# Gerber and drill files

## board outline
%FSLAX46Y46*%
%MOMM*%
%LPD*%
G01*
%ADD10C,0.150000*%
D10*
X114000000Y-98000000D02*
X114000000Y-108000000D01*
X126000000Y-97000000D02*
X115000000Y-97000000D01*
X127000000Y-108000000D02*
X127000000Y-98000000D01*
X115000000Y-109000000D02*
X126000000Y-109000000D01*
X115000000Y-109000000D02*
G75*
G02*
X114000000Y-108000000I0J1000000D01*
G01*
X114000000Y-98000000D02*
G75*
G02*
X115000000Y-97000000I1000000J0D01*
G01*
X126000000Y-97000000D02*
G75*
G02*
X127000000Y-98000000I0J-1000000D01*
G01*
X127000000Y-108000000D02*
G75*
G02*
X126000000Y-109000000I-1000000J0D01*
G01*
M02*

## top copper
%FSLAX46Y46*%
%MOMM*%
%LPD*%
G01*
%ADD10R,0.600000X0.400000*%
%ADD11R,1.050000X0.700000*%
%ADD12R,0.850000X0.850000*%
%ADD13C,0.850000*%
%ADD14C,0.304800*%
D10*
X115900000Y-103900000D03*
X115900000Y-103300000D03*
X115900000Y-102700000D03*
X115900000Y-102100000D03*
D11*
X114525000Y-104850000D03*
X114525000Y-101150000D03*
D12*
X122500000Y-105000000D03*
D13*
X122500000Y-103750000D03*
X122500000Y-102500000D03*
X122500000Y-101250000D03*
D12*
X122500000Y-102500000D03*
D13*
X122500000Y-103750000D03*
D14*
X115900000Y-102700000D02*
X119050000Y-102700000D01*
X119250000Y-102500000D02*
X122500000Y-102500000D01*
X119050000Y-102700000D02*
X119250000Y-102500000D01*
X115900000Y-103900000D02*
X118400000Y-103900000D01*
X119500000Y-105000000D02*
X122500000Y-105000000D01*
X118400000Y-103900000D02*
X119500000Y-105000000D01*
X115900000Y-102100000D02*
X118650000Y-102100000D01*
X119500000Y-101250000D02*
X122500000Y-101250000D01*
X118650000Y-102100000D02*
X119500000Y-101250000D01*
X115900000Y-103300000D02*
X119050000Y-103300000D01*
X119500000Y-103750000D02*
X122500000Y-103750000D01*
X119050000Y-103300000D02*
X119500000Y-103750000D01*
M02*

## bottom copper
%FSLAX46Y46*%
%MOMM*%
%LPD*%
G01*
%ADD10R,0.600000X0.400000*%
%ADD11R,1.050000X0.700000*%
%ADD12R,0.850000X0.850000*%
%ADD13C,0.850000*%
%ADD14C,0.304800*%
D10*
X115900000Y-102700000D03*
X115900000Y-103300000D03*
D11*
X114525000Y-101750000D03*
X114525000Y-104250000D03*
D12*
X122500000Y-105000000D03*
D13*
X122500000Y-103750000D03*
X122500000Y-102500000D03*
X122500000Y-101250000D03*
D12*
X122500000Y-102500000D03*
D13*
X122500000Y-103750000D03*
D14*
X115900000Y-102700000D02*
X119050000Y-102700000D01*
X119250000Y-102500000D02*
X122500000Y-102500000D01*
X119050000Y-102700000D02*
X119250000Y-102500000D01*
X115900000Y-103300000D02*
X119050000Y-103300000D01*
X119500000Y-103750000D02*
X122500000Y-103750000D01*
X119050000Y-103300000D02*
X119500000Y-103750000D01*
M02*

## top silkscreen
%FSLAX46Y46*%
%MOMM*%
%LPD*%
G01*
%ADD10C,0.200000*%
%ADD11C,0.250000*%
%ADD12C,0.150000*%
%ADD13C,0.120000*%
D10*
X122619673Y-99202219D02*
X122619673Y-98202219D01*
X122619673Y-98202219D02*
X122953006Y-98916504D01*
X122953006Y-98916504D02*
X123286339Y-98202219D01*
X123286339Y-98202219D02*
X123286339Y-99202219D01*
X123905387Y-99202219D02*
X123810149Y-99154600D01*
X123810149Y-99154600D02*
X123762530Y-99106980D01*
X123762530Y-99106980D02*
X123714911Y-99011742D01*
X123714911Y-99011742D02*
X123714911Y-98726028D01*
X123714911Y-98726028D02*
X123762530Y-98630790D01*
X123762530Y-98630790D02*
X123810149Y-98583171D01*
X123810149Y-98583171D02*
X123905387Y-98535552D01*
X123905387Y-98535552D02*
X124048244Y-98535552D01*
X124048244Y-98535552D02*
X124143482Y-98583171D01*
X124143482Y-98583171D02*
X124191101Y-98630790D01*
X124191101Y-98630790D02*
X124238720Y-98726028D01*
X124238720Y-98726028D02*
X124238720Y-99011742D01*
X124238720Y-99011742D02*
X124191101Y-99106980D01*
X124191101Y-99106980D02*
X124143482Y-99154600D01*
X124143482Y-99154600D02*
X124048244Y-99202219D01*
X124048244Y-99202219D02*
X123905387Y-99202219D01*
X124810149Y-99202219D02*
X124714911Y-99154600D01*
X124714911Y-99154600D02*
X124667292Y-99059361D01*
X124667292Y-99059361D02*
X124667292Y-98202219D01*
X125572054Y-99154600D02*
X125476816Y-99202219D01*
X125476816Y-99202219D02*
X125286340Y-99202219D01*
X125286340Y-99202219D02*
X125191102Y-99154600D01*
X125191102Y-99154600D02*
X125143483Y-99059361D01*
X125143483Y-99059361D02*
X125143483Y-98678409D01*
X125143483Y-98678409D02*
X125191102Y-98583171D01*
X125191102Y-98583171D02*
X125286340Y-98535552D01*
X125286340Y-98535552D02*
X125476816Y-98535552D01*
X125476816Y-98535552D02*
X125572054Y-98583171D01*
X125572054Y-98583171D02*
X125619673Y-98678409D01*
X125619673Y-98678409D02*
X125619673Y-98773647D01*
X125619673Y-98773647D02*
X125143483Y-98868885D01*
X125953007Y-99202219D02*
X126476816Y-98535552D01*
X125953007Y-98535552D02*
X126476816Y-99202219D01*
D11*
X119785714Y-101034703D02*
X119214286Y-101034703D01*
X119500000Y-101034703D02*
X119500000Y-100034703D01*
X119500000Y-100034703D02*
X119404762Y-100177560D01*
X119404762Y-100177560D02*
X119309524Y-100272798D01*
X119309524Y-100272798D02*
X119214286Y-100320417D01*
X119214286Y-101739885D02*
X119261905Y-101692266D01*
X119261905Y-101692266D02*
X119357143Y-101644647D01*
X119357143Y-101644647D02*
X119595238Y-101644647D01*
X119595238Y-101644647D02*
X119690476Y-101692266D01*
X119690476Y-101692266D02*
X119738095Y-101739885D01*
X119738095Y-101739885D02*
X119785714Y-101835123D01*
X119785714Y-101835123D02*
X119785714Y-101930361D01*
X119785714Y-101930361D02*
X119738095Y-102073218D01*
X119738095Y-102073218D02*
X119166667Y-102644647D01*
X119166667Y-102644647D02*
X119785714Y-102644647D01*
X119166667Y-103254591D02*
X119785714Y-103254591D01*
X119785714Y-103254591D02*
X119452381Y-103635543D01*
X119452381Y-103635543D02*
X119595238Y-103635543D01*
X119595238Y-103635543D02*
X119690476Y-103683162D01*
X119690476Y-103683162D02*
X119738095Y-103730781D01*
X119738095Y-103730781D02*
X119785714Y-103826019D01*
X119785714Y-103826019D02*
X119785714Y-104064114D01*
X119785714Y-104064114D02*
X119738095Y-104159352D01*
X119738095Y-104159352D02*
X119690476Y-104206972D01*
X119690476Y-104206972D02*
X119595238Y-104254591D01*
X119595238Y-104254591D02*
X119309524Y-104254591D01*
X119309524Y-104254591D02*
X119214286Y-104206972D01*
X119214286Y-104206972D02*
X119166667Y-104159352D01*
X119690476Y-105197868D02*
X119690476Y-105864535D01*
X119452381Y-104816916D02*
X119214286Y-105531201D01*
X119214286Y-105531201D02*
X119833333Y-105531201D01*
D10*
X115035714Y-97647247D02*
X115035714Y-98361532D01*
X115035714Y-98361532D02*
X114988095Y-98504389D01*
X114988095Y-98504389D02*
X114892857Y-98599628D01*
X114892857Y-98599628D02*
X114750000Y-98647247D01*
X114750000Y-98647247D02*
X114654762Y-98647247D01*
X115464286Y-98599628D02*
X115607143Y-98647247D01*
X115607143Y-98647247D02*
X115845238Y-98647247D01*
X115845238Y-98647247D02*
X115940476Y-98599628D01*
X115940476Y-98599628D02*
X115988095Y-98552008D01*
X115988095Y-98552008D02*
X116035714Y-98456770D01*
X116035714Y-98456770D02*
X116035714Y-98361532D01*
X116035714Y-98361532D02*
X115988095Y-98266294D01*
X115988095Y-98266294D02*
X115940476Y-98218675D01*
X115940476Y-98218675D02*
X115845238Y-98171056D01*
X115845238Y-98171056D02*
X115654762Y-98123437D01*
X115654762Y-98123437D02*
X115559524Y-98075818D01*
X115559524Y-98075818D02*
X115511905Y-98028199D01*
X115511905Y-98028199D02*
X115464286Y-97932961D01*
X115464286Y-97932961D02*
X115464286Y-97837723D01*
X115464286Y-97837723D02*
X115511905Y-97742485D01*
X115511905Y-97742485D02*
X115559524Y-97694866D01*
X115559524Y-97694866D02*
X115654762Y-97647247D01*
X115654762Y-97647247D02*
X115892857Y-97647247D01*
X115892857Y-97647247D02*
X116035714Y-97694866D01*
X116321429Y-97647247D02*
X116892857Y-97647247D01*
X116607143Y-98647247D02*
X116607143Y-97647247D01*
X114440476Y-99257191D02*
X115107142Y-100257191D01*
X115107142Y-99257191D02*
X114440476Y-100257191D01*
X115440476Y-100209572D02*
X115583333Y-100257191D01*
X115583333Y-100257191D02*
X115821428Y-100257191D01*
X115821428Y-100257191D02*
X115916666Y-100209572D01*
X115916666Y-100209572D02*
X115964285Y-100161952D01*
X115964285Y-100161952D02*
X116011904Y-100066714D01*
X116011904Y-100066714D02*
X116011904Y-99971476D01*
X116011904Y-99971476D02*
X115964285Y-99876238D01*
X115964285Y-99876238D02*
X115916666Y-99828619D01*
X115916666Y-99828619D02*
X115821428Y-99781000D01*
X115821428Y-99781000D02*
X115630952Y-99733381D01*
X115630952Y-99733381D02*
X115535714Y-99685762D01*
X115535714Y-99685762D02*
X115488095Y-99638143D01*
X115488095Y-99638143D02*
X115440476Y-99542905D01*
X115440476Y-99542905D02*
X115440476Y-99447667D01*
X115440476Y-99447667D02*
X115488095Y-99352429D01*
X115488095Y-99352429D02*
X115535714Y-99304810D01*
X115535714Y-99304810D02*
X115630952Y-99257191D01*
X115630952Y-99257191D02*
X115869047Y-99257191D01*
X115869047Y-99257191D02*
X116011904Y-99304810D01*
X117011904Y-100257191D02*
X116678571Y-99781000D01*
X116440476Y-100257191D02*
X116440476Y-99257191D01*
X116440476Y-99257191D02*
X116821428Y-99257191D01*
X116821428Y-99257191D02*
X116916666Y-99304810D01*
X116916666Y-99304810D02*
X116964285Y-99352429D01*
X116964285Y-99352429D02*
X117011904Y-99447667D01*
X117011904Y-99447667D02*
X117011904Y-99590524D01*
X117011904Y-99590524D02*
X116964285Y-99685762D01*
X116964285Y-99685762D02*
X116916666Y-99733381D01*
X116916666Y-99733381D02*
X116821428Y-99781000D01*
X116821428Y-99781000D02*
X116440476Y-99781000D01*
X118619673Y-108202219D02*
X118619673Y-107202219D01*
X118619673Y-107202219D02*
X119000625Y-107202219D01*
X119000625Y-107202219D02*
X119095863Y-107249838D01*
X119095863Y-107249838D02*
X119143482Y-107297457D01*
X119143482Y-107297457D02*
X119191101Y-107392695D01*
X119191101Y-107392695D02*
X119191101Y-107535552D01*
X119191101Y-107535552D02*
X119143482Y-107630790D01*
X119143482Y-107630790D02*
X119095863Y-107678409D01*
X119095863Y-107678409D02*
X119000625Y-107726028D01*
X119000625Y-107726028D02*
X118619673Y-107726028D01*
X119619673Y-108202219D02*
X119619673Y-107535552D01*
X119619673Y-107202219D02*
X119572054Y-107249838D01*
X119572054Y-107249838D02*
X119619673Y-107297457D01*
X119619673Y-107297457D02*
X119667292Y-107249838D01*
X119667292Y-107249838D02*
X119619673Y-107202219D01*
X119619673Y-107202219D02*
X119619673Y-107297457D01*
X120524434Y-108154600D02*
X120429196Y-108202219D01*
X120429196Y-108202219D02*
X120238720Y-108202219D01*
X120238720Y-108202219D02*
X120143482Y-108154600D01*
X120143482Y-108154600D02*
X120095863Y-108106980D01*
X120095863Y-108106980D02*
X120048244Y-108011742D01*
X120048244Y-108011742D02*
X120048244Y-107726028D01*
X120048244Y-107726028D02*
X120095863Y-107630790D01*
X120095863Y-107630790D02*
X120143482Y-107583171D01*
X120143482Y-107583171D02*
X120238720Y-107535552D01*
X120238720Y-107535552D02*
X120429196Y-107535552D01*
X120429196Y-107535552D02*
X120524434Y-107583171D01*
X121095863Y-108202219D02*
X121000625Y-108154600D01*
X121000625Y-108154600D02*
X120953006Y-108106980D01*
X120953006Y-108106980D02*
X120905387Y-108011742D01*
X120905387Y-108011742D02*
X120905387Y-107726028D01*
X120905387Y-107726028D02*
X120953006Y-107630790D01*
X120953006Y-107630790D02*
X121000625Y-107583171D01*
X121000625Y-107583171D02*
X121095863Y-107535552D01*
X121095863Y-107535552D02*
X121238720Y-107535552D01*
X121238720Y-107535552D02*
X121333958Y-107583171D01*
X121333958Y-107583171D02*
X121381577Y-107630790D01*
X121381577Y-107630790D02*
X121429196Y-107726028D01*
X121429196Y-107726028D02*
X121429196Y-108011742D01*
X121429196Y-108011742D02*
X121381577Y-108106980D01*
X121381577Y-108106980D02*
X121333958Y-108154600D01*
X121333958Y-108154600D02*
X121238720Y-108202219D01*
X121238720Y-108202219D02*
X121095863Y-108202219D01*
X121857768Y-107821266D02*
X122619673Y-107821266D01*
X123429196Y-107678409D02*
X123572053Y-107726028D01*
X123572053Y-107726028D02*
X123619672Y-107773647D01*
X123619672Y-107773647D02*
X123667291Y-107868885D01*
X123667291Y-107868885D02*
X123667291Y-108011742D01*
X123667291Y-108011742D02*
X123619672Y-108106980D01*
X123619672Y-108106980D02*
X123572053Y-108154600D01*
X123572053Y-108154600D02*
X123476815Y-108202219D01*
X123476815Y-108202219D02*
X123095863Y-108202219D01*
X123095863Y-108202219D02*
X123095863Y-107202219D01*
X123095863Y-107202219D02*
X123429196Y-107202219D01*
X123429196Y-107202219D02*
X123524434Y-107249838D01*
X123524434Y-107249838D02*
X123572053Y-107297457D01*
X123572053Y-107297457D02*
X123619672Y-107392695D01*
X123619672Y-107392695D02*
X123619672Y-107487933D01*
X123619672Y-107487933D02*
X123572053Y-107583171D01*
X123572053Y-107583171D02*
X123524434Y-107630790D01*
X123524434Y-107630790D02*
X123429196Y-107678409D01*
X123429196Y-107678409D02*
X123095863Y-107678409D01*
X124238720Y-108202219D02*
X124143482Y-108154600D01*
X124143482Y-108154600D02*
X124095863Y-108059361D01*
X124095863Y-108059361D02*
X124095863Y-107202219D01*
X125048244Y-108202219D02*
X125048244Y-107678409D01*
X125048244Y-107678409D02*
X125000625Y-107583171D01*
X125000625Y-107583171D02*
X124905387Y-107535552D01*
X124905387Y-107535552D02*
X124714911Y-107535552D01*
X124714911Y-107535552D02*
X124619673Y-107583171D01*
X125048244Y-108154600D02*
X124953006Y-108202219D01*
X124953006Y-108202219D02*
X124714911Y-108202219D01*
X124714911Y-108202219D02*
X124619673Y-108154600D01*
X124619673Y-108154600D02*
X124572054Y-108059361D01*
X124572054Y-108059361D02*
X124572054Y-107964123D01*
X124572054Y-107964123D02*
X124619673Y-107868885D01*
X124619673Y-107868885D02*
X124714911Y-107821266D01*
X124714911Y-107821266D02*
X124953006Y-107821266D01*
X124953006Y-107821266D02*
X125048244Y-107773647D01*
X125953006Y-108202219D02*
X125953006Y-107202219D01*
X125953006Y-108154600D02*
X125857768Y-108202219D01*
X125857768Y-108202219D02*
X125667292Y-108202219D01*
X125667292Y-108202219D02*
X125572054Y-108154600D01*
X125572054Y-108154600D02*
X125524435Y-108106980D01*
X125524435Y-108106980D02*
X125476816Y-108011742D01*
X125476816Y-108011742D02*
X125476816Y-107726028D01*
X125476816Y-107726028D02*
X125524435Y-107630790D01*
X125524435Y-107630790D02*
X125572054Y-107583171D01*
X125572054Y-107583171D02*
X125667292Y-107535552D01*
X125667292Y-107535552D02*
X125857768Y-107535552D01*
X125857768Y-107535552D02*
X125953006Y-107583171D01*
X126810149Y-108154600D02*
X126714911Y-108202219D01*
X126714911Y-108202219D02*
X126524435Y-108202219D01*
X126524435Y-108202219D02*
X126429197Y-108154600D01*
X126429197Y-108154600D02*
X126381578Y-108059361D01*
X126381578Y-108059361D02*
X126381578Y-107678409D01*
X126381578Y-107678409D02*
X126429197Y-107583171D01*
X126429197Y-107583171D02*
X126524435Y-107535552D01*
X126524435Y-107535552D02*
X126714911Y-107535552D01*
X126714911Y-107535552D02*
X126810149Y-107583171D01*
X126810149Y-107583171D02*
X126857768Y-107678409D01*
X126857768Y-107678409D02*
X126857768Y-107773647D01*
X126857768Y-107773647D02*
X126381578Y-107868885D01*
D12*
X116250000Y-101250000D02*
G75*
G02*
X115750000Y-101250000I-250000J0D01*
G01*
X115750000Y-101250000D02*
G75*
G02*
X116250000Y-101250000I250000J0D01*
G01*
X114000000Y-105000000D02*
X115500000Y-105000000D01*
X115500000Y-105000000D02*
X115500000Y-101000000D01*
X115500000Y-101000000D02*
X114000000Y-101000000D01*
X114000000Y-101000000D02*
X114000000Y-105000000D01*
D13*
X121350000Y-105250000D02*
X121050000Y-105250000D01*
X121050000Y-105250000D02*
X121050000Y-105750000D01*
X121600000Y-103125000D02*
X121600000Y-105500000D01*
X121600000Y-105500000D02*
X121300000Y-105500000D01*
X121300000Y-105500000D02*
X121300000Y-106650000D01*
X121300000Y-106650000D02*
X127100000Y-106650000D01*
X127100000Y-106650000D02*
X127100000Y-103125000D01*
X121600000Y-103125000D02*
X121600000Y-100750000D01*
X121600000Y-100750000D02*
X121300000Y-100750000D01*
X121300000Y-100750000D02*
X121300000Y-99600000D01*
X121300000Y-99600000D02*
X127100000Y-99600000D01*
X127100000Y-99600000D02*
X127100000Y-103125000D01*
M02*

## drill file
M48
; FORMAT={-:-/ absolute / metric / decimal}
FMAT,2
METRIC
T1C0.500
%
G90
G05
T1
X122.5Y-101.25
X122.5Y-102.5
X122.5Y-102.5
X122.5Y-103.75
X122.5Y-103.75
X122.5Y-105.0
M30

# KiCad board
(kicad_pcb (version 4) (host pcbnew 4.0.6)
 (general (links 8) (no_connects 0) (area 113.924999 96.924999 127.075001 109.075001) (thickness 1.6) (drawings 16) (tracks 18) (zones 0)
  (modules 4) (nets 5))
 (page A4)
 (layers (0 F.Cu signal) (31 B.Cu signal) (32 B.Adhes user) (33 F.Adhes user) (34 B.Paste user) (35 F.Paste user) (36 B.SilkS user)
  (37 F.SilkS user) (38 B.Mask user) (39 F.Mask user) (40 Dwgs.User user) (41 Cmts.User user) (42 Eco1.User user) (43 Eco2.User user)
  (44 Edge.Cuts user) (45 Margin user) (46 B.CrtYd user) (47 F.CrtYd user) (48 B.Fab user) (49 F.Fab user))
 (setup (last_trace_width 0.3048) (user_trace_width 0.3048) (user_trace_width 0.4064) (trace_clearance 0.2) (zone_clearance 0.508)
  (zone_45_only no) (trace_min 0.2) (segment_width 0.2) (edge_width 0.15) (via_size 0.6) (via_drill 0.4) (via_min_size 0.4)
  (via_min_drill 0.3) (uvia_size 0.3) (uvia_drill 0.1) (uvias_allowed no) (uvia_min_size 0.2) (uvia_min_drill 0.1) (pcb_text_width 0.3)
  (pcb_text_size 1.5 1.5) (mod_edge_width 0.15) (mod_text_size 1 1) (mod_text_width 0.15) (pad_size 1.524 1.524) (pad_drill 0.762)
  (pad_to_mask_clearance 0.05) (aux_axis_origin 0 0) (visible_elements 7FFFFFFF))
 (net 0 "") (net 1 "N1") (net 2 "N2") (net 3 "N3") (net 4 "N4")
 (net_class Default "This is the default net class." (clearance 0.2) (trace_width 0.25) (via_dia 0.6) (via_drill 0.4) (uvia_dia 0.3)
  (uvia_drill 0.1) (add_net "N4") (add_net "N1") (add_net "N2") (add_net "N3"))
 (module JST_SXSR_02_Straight (layer B.Cu) (at 114 103 270)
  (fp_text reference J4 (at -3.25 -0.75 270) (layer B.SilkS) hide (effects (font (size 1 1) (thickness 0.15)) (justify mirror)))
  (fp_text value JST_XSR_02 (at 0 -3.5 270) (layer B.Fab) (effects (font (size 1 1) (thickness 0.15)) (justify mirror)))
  (pad 2 smd rect (at -0.3 -1.9 270) (size 0.4 0.6) (layers B.Cu B.Paste B.Mask) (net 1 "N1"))
  (pad 1 smd rect (at 0.3 -1.9 270) (size 0.4 0.6) (layers B.Cu B.Paste B.Mask) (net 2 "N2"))
  (pad "" smd rect (at -1.25 -0.525 270) (size 0.7 1.05) (layers B.Cu B.Paste B.Mask))
  (pad "" smd rect (at 1.25 -0.525 270) (size 0.7 1.05) (layers B.Cu B.Paste B.Mask)))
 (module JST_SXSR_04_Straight (layer F.Cu) (at 114 103 90)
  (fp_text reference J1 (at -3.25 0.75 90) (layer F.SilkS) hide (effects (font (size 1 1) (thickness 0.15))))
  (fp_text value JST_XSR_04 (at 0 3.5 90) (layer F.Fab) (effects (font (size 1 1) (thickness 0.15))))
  (fp_circle (center 1.75 2) (end 1.75 1.75) (layer F.SilkS) (width 0.15))
  (fp_line (start -2 0) (end -2 1.5) (layer F.SilkS) (width 0.15))
  (fp_line (start -2 1.5) (end 2 1.5) (layer F.SilkS) (width 0.15))
  (fp_line (start 2 1.5) (end 2 0) (layer F.SilkS) (width 0.15))
  (fp_line (start 2 0) (end -2 0) (layer F.SilkS) (width 0.15))
  (pad 4 smd rect (at -0.9 1.9 90) (size 0.4 0.6) (layers F.Cu F.Paste F.Mask) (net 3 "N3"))
  (pad 3 smd rect (at -0.3 1.9 90) (size 0.4 0.6) (layers F.Cu F.Paste F.Mask) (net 2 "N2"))
  (pad 2 smd rect (at 0.3 1.9 90) (size 0.4 0.6) (layers F.Cu F.Paste F.Mask) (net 1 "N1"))
  (pad 1 smd rect (at 0.9 1.9 90) (size 0.4 0.6) (layers F.Cu F.Paste F.Mask) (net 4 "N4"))
  (pad "" smd rect (at -1.85 0.525 90) (size 0.7 1.05) (layers F.Cu F.Paste F.Mask))
  (pad "" smd rect (at 1.85 0.525 90) (size 0.7 1.05) (layers F.Cu F.Paste F.Mask)))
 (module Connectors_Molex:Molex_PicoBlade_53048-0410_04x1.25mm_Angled (layer F.Cu) (at 122.5 105 90)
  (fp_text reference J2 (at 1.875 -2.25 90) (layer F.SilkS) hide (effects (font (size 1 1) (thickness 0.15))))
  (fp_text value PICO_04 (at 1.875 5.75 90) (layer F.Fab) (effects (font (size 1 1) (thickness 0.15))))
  (fp_line (start -0.25 -1.15) (end -0.25 -1.45) (layer F.SilkS) (width 0.12))
  (fp_line (start -0.25 -1.45) (end -0.75 -1.45) (layer F.SilkS) (width 0.12))
  (fp_line (start 1.875 -0.9) (end -0.5 -0.9) (layer F.SilkS) (width 0.12))
  (fp_line (start -0.5 -0.9) (end -0.5 -1.2) (layer F.SilkS) (width 0.12))
  (fp_line (start -0.5 -1.2) (end -1.65 -1.2) (layer F.SilkS) (width 0.12))
  (fp_line (start -1.65 -1.2) (end -1.65 4.6) (layer F.SilkS) (width 0.12))
  (fp_line (start -1.65 4.6) (end 1.875 4.6) (layer F.SilkS) (width 0.12))
  (fp_line (start 1.875 -0.9) (end 4.25 -0.9) (layer F.SilkS) (width 0.12))
  (fp_line (start 4.25 -0.9) (end 4.25 -1.2) (layer F.SilkS) (width 0.12))
  (fp_line (start 4.25 -1.2) (end 5.4 -1.2) (layer F.SilkS) (width 0.12))
  (fp_line (start 5.4 -1.2) (end 5.4 4.6) (layer F.SilkS) (width 0.12))
  (fp_line (start 5.4 4.6) (end 1.875 4.6) (layer F.SilkS) (width 0.12))
  (pad 1 thru_hole rect (at 0 0 90) (size 0.85 0.85) (drill 0.5) (layers *.Cu *.Mask) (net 3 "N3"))
  (pad 2 thru_hole circle (at 1.25 0 90) (size 0.85 0.85) (drill 0.5) (layers *.Cu *.Mask) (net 2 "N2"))
  (pad 3 thru_hole circle (at 2.5 0 90) (size 0.85 0.85) (drill 0.5) (layers *.Cu *.Mask) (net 1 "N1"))
  (pad 4 thru_hole circle (at 3.75 0 90) (size 0.85 0.85) (drill 0.5) (layers *.Cu *.Mask) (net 4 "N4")))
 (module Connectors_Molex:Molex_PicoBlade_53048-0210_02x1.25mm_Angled (layer B.Cu) (at 122.5 102.5 270)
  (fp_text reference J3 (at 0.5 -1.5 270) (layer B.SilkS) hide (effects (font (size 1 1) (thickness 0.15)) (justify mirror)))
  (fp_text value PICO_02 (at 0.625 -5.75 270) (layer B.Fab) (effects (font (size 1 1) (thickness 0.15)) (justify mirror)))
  (pad 1 thru_hole rect (at 0 0 270) (size 0.85 0.85) (drill 0.5) (layers *.Cu *.Mask) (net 1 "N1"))
  (pad 2 thru_hole circle (at 1.25 0 270) (size 0.85 0.85) (drill 0.5) (layers *.Cu *.Mask) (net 2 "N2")))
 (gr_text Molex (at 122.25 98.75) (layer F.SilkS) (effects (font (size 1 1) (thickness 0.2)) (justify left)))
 (gr_line (start 114 98) (end 114 108) (angle 90) (layer Edge.Cuts) (width 0.15))
 (gr_line (start 126 97) (end 115 97) (angle 90) (layer Edge.Cuts) (width 0.15))
 (gr_line (start 127 108) (end 127 98) (angle 90) (layer Edge.Cuts) (width 0.15))
 (gr_line (start 115 109) (end 126 109) (angle 90) (layer Edge.Cuts) (width 0.15))
 (gr_arc (start 115 108) (end 115 109) (angle 90) (layer Edge.Cuts) (width 0.15))
 (gr_arc (start 115 98) (end 114 98) (angle 90) (layer Edge.Cuts) (width 0.15))
 (gr_arc (start 126 98) (end 126 97) (angle 90) (layer Edge.Cuts) (width 0.15))
 (gr_arc (start 126 108) (end 127 108) (angle 90) (layer Edge.Cuts) (width 0.15))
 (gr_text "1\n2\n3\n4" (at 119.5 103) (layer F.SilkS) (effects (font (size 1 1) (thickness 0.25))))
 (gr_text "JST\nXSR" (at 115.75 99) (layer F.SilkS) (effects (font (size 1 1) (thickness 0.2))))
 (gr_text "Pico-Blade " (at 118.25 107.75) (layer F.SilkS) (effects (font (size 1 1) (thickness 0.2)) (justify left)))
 (segment (start 115.9 102.7) (end 119.05 102.7) (width 0.3048) (layer B.Cu) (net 1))
 (segment (start 119.25 102.5) (end 122.5 102.5) (width 0.3048) (layer B.Cu) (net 1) (status 20))
 (segment (start 119.05 102.7) (end 119.25 102.5) (width 0.3048) (layer B.Cu) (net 1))
 (segment (start 115.9 102.7) (end 119.05 102.7) (width 0.3048) (layer F.Cu) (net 1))
 (segment (start 119.25 102.5) (end 122.5 102.5) (width 0.3048) (layer F.Cu) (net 1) (status 20))
 (segment (start 119.05 102.7) (end 119.25 102.5) (width 0.3048) (layer F.Cu) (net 1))
 (segment (start 115.9 103.9) (end 118.4 103.9) (width 0.3048) (layer F.Cu) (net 3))
 (segment (start 119.5 105) (end 122.5 105) (width 0.3048) (layer F.Cu) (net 3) (status 20))
 (segment (start 118.4 103.9) (end 119.5 105) (width 0.3048) (layer F.Cu) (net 3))
 (segment (start 115.9 102.1) (end 118.65 102.1) (width 0.3048) (layer F.Cu) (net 4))
 (segment (start 119.5 101.25) (end 122.5 101.25) (width 0.3048) (layer F.Cu) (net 4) (status 20))
 (segment (start 118.65 102.1) (end 119.5 101.25) (width 0.3048) (layer F.Cu) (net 4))
 (segment (start 115.9 103.3) (end 119.05 103.3) (width 0.3048) (layer B.Cu) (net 2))
 (segment (start 119.5 103.75) (end 122.5 103.75) (width 0.3048) (layer B.Cu) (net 2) (status 20))
 (segment (start 119.05 103.3) (end 119.5 103.75) (width 0.3048) (layer B.Cu) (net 2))
 (segment (start 115.9 103.3) (end 119.05 103.3) (width 0.3048) (layer F.Cu) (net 2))
 (segment (start 119.5 103.75) (end 122.5 103.75) (width 0.3048) (layer F.Cu) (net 2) (status 20))
 (segment (start 119.05 103.3) (end 119.5 103.75) (width 0.3048) (layer F.Cu) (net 2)))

